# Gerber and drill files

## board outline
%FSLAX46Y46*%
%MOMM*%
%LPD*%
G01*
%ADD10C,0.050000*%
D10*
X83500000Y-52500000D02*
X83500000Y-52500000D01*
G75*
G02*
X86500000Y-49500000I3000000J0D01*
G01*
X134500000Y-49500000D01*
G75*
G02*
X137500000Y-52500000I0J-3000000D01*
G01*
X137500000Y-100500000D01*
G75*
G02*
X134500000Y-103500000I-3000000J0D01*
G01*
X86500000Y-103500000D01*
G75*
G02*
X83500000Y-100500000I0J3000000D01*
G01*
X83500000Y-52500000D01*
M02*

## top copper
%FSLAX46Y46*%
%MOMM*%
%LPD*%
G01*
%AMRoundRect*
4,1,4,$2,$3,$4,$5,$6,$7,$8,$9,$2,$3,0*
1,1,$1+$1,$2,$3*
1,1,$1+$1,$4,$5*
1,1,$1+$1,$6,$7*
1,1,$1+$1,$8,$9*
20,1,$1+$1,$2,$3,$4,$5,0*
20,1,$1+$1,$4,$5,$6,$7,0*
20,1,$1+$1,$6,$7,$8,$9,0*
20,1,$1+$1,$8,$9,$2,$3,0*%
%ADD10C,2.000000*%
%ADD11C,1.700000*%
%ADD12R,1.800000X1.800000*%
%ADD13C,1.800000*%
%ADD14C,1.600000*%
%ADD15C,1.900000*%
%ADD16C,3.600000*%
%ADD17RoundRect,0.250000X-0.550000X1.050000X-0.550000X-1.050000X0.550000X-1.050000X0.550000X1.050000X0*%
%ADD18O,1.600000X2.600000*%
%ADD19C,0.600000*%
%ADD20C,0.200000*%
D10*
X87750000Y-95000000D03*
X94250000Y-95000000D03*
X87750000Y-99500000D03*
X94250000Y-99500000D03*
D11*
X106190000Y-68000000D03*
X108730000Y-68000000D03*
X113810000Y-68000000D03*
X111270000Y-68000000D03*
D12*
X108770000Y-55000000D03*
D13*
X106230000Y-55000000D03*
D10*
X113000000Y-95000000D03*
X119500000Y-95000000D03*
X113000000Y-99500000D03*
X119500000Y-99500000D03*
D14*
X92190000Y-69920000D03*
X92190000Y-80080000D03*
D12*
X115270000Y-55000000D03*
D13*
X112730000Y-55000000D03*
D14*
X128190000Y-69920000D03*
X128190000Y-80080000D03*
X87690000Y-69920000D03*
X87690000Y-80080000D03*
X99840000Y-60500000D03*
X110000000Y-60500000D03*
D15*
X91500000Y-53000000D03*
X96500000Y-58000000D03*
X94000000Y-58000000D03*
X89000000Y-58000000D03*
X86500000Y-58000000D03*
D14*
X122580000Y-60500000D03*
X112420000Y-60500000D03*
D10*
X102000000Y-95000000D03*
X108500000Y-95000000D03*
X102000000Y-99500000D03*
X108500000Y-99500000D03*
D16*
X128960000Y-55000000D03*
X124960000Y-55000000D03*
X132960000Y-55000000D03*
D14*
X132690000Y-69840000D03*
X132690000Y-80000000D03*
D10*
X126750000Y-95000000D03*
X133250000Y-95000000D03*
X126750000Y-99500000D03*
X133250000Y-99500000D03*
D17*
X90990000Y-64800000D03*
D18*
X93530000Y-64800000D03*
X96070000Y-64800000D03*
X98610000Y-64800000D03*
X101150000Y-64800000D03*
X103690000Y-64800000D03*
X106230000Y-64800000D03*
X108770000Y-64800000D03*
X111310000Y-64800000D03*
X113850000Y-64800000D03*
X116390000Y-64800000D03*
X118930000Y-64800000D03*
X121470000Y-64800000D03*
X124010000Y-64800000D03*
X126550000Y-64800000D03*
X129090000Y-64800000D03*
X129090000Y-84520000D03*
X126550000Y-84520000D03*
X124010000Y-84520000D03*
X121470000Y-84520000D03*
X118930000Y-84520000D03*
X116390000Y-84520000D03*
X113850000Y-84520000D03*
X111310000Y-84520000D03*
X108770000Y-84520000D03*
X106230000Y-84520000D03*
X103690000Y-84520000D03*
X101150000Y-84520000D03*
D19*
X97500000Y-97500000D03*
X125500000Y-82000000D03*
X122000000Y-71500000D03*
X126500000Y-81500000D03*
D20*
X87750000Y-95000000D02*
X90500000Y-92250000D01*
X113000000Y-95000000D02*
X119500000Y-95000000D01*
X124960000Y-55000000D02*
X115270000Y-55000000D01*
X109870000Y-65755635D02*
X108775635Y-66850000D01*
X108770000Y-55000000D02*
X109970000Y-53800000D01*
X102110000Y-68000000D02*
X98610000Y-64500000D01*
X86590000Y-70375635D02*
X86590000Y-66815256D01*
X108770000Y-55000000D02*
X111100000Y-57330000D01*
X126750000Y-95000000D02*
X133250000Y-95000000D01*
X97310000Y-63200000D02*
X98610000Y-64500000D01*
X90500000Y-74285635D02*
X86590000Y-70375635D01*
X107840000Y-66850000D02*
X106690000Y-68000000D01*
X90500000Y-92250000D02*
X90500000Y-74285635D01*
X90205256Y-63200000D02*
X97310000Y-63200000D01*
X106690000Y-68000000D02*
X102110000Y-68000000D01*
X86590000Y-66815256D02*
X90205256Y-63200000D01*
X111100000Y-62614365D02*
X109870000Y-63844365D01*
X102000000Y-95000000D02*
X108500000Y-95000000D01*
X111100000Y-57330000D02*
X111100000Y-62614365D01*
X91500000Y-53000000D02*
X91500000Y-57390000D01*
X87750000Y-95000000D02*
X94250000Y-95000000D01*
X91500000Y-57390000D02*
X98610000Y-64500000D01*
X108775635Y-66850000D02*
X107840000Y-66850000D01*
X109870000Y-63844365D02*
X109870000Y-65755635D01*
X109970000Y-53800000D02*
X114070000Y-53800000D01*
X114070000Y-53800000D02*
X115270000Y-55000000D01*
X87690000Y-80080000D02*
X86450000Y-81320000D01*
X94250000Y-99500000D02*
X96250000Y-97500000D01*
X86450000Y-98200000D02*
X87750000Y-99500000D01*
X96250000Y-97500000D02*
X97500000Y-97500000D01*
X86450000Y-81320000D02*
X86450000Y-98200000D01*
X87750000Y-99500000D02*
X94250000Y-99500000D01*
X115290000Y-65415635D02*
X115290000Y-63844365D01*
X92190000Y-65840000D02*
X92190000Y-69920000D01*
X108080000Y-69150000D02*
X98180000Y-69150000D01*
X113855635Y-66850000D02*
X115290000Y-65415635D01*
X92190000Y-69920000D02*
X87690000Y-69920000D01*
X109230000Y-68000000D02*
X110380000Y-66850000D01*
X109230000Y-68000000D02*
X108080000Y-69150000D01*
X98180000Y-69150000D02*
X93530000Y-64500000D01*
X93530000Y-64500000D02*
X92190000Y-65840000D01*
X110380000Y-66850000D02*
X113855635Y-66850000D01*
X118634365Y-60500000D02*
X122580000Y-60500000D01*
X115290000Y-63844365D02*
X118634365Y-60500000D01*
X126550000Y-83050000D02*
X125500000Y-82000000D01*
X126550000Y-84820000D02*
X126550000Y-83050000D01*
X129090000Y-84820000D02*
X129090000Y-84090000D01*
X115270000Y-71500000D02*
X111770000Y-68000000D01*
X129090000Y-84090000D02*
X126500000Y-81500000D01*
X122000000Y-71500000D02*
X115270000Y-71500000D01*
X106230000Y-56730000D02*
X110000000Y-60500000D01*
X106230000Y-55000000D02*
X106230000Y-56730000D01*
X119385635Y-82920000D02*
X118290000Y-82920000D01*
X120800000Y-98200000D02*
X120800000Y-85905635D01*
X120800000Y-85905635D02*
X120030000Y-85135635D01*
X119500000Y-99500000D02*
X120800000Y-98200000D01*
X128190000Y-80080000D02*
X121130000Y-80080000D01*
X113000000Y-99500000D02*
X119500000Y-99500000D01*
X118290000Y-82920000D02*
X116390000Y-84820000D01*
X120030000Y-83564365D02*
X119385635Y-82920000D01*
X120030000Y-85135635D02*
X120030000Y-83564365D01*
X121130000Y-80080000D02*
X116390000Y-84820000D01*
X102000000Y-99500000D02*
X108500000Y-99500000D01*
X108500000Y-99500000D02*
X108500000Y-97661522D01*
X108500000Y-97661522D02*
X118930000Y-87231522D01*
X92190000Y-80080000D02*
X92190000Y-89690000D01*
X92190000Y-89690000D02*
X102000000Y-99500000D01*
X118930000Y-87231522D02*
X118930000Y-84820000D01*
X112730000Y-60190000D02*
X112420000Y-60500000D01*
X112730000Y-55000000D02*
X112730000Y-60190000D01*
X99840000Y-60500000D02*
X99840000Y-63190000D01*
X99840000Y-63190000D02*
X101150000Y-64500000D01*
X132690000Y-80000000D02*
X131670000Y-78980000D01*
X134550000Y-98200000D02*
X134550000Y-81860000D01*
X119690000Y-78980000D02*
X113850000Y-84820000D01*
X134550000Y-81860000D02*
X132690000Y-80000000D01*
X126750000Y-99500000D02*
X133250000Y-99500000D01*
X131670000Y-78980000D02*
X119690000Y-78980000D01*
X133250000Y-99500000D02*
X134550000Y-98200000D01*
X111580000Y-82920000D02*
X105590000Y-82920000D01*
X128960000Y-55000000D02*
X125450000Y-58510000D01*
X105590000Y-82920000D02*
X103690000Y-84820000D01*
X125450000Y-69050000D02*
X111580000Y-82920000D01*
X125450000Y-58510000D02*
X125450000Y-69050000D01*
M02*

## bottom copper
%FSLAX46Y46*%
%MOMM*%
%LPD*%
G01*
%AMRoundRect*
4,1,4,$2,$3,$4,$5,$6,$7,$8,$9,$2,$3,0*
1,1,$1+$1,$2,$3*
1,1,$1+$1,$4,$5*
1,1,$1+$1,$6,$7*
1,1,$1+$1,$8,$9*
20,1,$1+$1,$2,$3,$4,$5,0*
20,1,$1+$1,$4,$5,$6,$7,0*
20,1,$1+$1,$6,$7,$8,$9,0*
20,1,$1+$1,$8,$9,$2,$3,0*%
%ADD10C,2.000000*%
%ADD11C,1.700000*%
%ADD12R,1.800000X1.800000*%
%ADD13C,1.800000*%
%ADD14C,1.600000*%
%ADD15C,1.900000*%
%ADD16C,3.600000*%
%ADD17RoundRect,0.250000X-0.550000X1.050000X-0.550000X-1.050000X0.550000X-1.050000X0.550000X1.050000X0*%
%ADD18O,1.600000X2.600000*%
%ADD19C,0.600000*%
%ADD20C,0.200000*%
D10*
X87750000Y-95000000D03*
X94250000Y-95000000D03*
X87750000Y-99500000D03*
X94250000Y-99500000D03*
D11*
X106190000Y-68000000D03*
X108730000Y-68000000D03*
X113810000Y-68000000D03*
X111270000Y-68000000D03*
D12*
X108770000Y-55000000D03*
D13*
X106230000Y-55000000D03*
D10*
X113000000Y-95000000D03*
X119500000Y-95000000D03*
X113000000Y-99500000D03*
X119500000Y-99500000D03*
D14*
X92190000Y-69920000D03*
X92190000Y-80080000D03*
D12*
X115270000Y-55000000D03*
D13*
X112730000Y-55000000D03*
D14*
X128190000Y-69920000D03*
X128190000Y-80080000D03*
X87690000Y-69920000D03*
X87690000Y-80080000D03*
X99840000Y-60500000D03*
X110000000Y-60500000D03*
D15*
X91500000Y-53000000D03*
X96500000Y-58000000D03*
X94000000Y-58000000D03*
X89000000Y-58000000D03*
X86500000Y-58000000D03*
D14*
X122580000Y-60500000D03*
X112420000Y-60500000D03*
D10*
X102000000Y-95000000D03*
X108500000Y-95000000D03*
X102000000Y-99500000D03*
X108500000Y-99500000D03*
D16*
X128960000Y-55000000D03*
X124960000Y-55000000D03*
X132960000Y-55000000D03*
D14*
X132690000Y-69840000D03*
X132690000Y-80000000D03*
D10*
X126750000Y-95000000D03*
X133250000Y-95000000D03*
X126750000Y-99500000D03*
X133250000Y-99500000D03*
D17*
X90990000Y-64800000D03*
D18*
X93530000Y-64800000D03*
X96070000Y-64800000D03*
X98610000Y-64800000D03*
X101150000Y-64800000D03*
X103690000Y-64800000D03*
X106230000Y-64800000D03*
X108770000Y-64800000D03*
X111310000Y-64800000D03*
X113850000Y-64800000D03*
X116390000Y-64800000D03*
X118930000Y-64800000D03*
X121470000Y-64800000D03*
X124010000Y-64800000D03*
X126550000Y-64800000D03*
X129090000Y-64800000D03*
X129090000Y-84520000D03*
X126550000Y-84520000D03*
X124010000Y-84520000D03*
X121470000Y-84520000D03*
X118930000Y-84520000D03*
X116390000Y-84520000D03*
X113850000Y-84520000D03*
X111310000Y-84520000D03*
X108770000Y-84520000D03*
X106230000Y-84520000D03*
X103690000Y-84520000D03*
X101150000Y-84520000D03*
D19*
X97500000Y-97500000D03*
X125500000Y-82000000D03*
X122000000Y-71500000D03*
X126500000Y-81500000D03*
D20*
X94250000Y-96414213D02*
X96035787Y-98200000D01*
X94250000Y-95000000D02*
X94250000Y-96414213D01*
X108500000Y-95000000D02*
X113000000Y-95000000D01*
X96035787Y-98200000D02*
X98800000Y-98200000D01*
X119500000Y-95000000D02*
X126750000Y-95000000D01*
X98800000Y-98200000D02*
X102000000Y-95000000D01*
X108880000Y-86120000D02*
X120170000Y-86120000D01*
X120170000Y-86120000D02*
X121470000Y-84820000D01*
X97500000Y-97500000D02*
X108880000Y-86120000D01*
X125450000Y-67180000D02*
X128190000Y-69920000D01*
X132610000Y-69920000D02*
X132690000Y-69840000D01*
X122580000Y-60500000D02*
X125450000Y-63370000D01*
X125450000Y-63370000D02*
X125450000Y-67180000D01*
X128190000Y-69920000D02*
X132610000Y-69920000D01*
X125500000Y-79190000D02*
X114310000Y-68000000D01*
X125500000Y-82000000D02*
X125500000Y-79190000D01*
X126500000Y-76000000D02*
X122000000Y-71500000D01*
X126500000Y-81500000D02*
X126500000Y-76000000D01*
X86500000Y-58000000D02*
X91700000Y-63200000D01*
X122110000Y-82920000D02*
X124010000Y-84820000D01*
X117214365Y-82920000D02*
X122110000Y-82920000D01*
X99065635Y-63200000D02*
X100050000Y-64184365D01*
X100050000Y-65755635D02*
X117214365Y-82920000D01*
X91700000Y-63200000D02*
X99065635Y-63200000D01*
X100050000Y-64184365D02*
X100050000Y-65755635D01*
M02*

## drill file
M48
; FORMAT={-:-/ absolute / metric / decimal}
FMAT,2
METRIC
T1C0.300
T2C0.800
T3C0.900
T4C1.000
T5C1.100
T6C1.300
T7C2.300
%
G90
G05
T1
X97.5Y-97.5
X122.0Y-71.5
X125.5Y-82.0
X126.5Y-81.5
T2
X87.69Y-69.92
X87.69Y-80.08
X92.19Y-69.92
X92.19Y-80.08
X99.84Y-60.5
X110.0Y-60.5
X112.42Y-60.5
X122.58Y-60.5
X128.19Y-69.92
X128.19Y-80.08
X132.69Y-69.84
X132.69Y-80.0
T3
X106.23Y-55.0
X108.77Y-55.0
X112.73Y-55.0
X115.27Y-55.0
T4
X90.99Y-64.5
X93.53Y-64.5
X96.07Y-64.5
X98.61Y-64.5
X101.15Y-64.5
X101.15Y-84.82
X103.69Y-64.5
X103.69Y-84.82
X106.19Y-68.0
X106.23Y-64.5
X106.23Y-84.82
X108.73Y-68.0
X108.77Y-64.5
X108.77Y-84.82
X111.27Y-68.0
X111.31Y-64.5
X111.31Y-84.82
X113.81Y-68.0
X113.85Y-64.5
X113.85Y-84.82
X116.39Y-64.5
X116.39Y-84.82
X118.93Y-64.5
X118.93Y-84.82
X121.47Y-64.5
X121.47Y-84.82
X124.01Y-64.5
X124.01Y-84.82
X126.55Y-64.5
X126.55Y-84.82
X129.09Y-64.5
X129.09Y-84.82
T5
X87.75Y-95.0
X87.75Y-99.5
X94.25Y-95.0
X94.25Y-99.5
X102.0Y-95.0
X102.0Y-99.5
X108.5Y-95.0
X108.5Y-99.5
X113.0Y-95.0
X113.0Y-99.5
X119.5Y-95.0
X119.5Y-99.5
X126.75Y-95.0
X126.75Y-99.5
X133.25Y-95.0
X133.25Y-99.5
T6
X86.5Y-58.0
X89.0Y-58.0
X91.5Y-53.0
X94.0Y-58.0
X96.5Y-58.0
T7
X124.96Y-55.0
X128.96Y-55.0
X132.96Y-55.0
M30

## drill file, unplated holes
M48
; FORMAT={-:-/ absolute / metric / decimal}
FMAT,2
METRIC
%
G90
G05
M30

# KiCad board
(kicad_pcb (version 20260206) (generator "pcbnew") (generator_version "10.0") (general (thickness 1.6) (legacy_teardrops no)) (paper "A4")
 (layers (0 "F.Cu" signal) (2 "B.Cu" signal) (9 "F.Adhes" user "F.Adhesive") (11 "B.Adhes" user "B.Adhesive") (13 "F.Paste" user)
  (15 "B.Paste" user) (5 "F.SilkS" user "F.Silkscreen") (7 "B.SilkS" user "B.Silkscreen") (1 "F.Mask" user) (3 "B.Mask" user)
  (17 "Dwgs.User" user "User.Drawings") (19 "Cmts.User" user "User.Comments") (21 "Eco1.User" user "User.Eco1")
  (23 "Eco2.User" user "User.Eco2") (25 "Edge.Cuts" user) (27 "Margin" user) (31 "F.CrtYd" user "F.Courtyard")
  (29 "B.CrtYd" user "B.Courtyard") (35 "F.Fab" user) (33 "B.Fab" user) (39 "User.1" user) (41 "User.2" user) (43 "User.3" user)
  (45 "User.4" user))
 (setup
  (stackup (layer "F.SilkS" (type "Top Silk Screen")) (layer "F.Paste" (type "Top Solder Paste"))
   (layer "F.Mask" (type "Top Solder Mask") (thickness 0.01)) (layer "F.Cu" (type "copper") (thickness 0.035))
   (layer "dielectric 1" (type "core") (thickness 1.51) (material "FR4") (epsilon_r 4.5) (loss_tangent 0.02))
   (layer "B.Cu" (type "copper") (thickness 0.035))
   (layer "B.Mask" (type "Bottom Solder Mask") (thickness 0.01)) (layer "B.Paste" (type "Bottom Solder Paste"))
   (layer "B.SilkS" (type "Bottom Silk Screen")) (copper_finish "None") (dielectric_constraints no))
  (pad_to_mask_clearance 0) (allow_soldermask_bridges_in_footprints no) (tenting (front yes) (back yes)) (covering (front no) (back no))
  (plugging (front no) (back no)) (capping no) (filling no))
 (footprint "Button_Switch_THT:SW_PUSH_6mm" (layer "F.Cu") (at 87.75 95)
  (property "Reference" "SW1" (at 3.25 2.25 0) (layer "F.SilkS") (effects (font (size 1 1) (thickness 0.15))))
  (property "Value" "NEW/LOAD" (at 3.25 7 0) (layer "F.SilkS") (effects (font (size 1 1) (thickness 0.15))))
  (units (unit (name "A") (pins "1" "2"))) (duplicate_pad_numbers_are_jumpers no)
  (pad "1" thru_hole circle (at 0 0 90) (size 2 2) (drill 1.1) (layers "*.Cu" "*.Mask") (remove_unused_layers no) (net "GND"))
  (pad "1" thru_hole circle (at 6.5 0 90) (size 2 2) (drill 1.1) (layers "*.Cu" "*.Mask") (remove_unused_layers no) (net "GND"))
  (pad "2" thru_hole circle (at 0 4.5 90) (size 2 2) (drill 1.1) (layers "*.Cu" "*.Mask") (remove_unused_layers no) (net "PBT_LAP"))
  (pad "2" thru_hole circle (at 6.5 4.5 90) (size 2 2) (drill 1.1) (layers "*.Cu" "*.Mask") (remove_unused_layers no) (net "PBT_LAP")))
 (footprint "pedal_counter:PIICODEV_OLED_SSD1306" (layer "F.Cu") (at 110 80)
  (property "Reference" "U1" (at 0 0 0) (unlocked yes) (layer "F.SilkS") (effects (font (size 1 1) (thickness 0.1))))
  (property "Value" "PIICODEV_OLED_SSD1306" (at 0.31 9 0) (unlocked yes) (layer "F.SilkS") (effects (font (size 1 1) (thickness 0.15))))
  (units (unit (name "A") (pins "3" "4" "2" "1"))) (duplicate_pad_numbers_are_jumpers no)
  (pad "1" thru_hole circle (at -3.81 -12) (size 1.7 1.7) (drill 1) (layers "*.Cu" "*.Mask") (remove_unused_layers no) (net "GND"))
  (pad "2" thru_hole circle (at -1.27 -12) (size 1.7 1.7) (drill 1) (layers "*.Cu" "*.Mask") (remove_unused_layers no) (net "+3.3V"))
  (pad "3" thru_hole circle (at 3.81 -12) (size 1.7 1.7) (drill 1) (layers "*.Cu" "*.Mask") (remove_unused_layers no) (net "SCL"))
  (pad "4" thru_hole circle (at 1.27 -12) (size 1.7 1.7) (drill 1) (layers "*.Cu" "*.Mask") (remove_unused_layers no) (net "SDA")))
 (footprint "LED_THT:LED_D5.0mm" (layer "F.Cu") (at 108.77 55 180)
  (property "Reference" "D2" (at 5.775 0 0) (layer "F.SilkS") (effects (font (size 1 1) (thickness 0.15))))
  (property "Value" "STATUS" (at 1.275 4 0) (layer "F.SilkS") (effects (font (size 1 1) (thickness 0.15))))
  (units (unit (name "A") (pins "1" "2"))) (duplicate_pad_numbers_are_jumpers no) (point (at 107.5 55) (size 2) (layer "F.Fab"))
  (pad "1" thru_hole rect (at 0 0 180) (size 1.8 1.8) (drill 0.9) (layers "*.Cu" "*.Mask") (remove_unused_layers no) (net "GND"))
  (pad "2" thru_hole circle (at 2.54 0 180) (size 1.8 1.8) (drill 0.9) (layers "*.Cu" "*.Mask") (remove_unused_layers no) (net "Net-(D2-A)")))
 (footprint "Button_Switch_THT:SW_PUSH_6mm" (layer "F.Cu") (at 113 95)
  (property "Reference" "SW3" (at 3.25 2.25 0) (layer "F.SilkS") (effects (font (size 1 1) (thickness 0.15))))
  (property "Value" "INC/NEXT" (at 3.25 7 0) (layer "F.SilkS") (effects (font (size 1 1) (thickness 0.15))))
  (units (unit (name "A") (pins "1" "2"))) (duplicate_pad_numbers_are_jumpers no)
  (pad "1" thru_hole circle (at 0 0 90) (size 2 2) (drill 1.1) (layers "*.Cu" "*.Mask") (remove_unused_layers no) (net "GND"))
  (pad "1" thru_hole circle (at 6.5 0 90) (size 2 2) (drill 1.1) (layers "*.Cu" "*.Mask") (remove_unused_layers no) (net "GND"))
  (pad "2" thru_hole circle (at 0 4.5 90) (size 2 2) (drill 1.1) (layers "*.Cu" "*.Mask") (remove_unused_layers no) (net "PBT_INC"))
  (pad "2" thru_hole circle (at 6.5 4.5 90) (size 2 2) (drill 1.1) (layers "*.Cu" "*.Mask") (remove_unused_layers no) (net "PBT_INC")))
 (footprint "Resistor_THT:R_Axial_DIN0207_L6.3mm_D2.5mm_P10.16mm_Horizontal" (layer "F.Cu") (at 92.19 69.92 -90)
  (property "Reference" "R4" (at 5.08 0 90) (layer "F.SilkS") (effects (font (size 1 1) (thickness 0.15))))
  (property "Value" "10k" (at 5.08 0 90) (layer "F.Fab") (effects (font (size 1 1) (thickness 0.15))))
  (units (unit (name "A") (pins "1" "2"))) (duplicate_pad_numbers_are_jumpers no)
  (pad "1" thru_hole circle (at 0 0 270) (size 1.6 1.6) (drill 0.8) (layers "*.Cu" "*.Mask") (remove_unused_layers no) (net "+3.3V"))
  (pad "2" thru_hole circle (at 10.16 0 270) (size 1.6 1.6) (drill 0.8) (layers "*.Cu" "*.Mask") (remove_unused_layers no) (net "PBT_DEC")))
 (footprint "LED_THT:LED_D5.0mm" (layer "F.Cu") (at 115.27 55 180)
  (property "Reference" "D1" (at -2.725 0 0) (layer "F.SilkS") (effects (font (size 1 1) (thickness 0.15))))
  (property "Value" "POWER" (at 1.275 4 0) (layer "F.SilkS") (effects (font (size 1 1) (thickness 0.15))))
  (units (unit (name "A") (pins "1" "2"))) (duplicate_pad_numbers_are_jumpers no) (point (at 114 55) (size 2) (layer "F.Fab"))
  (pad "1" thru_hole rect (at 0 0 180) (size 1.8 1.8) (drill 0.9) (layers "*.Cu" "*.Mask") (remove_unused_layers no) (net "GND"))
  (pad "2" thru_hole circle (at 2.54 0 180) (size 1.8 1.8) (drill 0.9) (layers "*.Cu" "*.Mask") (remove_unused_layers no) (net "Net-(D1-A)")))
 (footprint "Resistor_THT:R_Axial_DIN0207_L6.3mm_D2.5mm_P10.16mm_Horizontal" (layer "F.Cu") (at 128.19 69.92 -90)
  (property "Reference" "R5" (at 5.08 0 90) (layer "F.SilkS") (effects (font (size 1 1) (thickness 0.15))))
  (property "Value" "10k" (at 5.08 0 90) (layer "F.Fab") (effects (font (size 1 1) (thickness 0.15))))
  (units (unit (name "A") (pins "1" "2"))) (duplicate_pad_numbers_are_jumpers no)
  (pad "1" thru_hole circle (at 0 0 270) (size 1.6 1.6) (drill 0.8) (layers "*.Cu" "*.Mask") (remove_unused_layers no) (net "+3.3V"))
  (pad "2" thru_hole circle (at 10.16 0 270) (size 1.6 1.6) (drill 0.8) (layers "*.Cu" "*.Mask") (remove_unused_layers no) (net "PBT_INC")))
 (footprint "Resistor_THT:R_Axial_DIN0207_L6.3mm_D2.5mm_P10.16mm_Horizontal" (layer "F.Cu") (at 87.69 69.92 -90)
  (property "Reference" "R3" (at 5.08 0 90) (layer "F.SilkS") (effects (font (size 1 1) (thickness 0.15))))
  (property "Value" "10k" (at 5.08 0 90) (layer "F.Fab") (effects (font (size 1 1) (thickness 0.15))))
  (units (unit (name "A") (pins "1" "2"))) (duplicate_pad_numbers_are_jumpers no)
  (pad "1" thru_hole circle (at 0 0 270) (size 1.6 1.6) (drill 0.8) (layers "*.Cu" "*.Mask") (remove_unused_layers no) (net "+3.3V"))
  (pad "2" thru_hole circle (at 10.16 0 270) (size 1.6 1.6) (drill 0.8) (layers "*.Cu" "*.Mask") (remove_unused_layers no) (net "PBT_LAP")))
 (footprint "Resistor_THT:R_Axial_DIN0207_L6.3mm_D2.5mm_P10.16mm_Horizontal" (layer "F.Cu") (at 99.84 60.5)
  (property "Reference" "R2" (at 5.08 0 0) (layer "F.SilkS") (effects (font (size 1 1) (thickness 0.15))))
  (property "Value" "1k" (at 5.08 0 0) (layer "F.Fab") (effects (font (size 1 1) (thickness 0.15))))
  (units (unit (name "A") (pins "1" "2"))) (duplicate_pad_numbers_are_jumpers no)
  (pad "1" thru_hole circle (at 0 0) (size 1.6 1.6) (drill 0.8) (layers "*.Cu" "*.Mask") (remove_unused_layers no) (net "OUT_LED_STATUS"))
  (pad "2" thru_hole circle (at 10.16 0) (size 1.6 1.6) (drill 0.8) (layers "*.Cu" "*.Mask") (remove_unused_layers no) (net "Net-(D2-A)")))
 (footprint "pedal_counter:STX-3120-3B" (layer "F.Cu") (at 91.5 58 -90)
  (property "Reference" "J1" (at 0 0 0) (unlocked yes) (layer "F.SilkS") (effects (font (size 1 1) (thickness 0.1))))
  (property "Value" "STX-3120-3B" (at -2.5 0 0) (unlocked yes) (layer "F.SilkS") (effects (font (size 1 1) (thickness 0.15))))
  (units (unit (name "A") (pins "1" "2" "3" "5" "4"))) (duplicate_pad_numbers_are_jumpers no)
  (pad "1" thru_hole circle (at -5 0 270) (size 1.9 1.9) (drill 1.3) (layers "*.Cu" "*.Mask") (remove_unused_layers no) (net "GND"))
  (pad "2" thru_hole circle (at 0 -5 270) (size 1.9 1.9) (drill 1.3) (layers "*.Cu" "*.Mask") (remove_unused_layers no)
   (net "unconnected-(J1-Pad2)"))
  (pad "3" thru_hole circle (at 0 -2.5 270) (size 1.9 1.9) (drill 1.3) (layers "*.Cu" "*.Mask") (remove_unused_layers no)
   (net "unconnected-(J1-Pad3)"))
  (pad "4" thru_hole circle (at 0 2.5 270) (size 1.9 1.9) (drill 1.3) (layers "*.Cu" "*.Mask") (remove_unused_layers no)
   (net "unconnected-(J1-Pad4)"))
  (pad "5" thru_hole circle (at 0 5 270) (size 1.9 1.9) (drill 1.3) (layers "*.Cu" "*.Mask") (remove_unused_layers no) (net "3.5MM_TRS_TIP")))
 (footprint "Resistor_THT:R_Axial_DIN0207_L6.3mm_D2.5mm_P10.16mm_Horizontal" (layer "F.Cu") (at 122.58 60.5 180)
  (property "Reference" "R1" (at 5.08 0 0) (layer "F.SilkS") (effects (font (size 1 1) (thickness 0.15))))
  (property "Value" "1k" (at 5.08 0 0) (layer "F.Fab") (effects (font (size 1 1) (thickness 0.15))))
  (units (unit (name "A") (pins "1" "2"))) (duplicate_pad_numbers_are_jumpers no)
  (pad "1" thru_hole circle (at 0 0 180) (size 1.6 1.6) (drill 0.8) (layers "*.Cu" "*.Mask") (remove_unused_layers no) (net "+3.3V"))
  (pad "2" thru_hole circle (at 10.16 0 180) (size 1.6 1.6) (drill 0.8) (layers "*.Cu" "*.Mask") (remove_unused_layers no)
   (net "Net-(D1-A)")))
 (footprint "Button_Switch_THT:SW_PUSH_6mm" (layer "F.Cu") (at 102 95)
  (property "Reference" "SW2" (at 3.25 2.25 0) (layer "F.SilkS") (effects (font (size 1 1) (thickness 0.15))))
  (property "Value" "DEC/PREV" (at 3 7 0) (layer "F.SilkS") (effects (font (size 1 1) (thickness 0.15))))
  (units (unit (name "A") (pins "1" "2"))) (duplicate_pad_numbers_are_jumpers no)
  (pad "1" thru_hole circle (at 0 0 90) (size 2 2) (drill 1.1) (layers "*.Cu" "*.Mask") (remove_unused_layers no) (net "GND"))
  (pad "1" thru_hole circle (at 6.5 0 90) (size 2 2) (drill 1.1) (layers "*.Cu" "*.Mask") (remove_unused_layers no) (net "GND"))
  (pad "2" thru_hole circle (at 0 4.5 90) (size 2 2) (drill 1.1) (layers "*.Cu" "*.Mask") (remove_unused_layers no) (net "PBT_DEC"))
  (pad "2" thru_hole circle (at 6.5 4.5 90) (size 2 2) (drill 1.1) (layers "*.Cu" "*.Mask") (remove_unused_layers no) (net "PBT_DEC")))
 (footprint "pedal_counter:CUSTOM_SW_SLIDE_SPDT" (layer "F.Cu") (at 128.96 55)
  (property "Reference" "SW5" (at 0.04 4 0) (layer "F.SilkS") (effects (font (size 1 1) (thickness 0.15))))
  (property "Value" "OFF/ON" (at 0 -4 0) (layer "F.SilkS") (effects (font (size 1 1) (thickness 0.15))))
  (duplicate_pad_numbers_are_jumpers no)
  (pad "1" thru_hole circle (at 0 0) (size 3.6 3.6) (drill 2.3) (layers "*.Cu" "*.Mask") (remove_unused_layers no) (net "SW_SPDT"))
  (pad "2" thru_hole circle (at -4 0) (size 3.6 3.6) (drill 2.3) (layers "*.Cu" "*.Mask") (remove_unused_layers no) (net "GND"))
  (pad "3" thru_hole circle (at 4 0) (size 3.6 3.6) (drill 2.3) (layers "*.Cu" "*.Mask") (remove_unused_layers no)
   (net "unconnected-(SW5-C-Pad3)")))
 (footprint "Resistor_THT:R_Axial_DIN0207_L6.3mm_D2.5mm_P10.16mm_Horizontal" (layer "F.Cu") (at 132.69 69.84 -90)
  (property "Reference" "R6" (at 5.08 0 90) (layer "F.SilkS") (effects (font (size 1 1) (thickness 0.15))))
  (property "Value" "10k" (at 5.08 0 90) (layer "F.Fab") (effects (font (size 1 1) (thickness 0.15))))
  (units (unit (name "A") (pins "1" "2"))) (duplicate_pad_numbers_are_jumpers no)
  (pad "1" thru_hole circle (at 0 0 270) (size 1.6 1.6) (drill 0.8) (layers "*.Cu" "*.Mask") (remove_unused_layers no) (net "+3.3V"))
  (pad "2" thru_hole circle (at 10.16 0 270) (size 1.6 1.6) (drill 0.8) (layers "*.Cu" "*.Mask") (remove_unused_layers no) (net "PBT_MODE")))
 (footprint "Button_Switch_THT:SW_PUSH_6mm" (layer "F.Cu") (at 126.75 95)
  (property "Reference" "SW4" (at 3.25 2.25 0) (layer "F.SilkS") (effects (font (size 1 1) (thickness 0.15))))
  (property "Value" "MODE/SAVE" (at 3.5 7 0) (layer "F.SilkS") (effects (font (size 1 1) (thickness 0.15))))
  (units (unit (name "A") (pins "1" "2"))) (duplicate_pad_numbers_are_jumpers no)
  (pad "1" thru_hole circle (at 0 0 90) (size 2 2) (drill 1.1) (layers "*.Cu" "*.Mask") (remove_unused_layers no) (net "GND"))
  (pad "1" thru_hole circle (at 6.5 0 90) (size 2 2) (drill 1.1) (layers "*.Cu" "*.Mask") (remove_unused_layers no) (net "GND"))
  (pad "2" thru_hole circle (at 0 4.5 90) (size 2 2) (drill 1.1) (layers "*.Cu" "*.Mask") (remove_unused_layers no) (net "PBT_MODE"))
  (pad "2" thru_hole circle (at 6.5 4.5 90) (size 2 2) (drill 1.1) (layers "*.Cu" "*.Mask") (remove_unused_layers no) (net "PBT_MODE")))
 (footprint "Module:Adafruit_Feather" (layer "B.Cu") (at 90.99 64.5 -90)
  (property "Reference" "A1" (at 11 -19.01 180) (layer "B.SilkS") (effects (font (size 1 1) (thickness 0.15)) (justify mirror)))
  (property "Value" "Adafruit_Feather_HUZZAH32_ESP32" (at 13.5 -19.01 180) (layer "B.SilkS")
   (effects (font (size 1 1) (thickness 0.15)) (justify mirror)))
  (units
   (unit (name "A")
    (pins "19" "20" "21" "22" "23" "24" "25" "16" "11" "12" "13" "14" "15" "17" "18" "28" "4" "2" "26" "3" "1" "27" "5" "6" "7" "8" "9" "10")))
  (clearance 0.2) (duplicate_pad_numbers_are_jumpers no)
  (pad "1" thru_hole roundrect (at 0 0 270) (size 2.6 1.6) (drill 1 (offset 0.3 0)) (layers "*.Cu" "*.Mask") (remove_unused_layers no)
   (roundrect_rratio 0.15625) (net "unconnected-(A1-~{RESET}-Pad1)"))
  (pad "2" thru_hole oval (at 0 -2.54 270) (size 2.6 1.6) (drill 1 (offset 0.3 0)) (layers "*.Cu" "*.Mask") (remove_unused_layers no)
   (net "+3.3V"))
  (pad "3" thru_hole oval (at 0 -5.08 270) (size 2.6 1.6) (drill 1 (offset 0.3 0)) (layers "*.Cu" "*.Mask") (remove_unused_layers no)
   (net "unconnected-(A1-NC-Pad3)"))
  (pad "4" thru_hole oval (at 0 -7.62 270) (size 2.6 1.6) (drill 1 (offset 0.3 0)) (layers "*.Cu" "*.Mask") (remove_unused_layers no)
   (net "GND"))
  (pad "5" thru_hole oval (at 0 -10.16 270) (size 2.6 1.6) (drill 1 (offset 0.3 0)) (layers "*.Cu" "*.Mask") (remove_unused_layers no)
   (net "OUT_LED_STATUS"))
  (pad "6" thru_hole oval (at 0 -12.7 270) (size 2.6 1.6) (drill 1 (offset 0.3 0)) (layers "*.Cu" "*.Mask") (remove_unused_layers no)
   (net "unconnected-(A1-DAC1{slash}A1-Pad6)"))
  (pad "7" thru_hole oval (at 0 -15.24 270) (size 2.6 1.6) (drill 1 (offset 0.3 0)) (layers "*.Cu" "*.Mask") (remove_unused_layers no)
   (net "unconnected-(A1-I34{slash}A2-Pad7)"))
  (pad "8" thru_hole oval (at 0 -17.78 270) (size 2.6 1.6) (drill 1 (offset 0.3 0)) (layers "*.Cu" "*.Mask") (remove_unused_layers no)
   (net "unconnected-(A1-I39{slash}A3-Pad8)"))
  (pad "9" thru_hole oval (at 0 -20.32 270) (size 2.6 1.6) (drill 1 (offset 0.3 0)) (layers "*.Cu" "*.Mask") (remove_unused_layers no)
   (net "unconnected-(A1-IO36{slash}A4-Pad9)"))
  (pad "10" thru_hole oval (at 0 -22.86 270) (size 2.6 1.6) (drill 1 (offset 0.3 0)) (layers "*.Cu" "*.Mask") (remove_unused_layers no)
   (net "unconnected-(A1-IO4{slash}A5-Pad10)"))
  (pad "11" thru_hole oval (at 0 -25.4 270) (size 2.6 1.6) (drill 1 (offset 0.3 0)) (layers "*.Cu" "*.Mask") (remove_unused_layers no)
   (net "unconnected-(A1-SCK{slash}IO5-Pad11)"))
  (pad "12" thru_hole oval (at 0 -27.94 270) (size 2.6 1.6) (drill 1 (offset 0.3 0)) (layers "*.Cu" "*.Mask") (remove_unused_layers no)
   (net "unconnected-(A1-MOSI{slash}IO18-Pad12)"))
  (pad "13" thru_hole oval (at 0 -30.48 270) (size 2.6 1.6) (drill 1 (offset 0.3 0)) (layers "*.Cu" "*.Mask") (remove_unused_layers no)
   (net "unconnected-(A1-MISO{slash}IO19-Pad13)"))
  (pad "14" thru_hole oval (at 0 -33.02 270) (size 2.6 1.6) (drill 1 (offset 0.3 0)) (layers "*.Cu" "*.Mask") (remove_unused_layers no)
   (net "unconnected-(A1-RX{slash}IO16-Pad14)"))
  (pad "15" thru_hole oval (at 0 -35.56 270) (size 2.6 1.6) (drill 1 (offset 0.3 0)) (layers "*.Cu" "*.Mask") (remove_unused_layers no)
   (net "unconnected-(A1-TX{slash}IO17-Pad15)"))
  (pad "16" thru_hole oval (at 0 -38.1 270) (size 2.6 1.6) (drill 1 (offset 0.3 0)) (layers "*.Cu" "*.Mask") (remove_unused_layers no)
   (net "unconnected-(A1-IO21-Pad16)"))
  (pad "17" thru_hole oval (at 20.32 -38.1 90) (size 2.6 1.6) (drill 1 (offset 0.3 0)) (layers "*.Cu" "*.Mask") (remove_unused_layers no)
   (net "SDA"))
  (pad "18" thru_hole oval (at 20.32 -35.56 90) (size 2.6 1.6) (drill 1 (offset 0.3 0)) (layers "*.Cu" "*.Mask") (remove_unused_layers no)
   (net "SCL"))
  (pad "19" thru_hole oval (at 20.32 -33.02 90) (size 2.6 1.6) (drill 1 (offset 0.3 0)) (layers "*.Cu" "*.Mask") (remove_unused_layers no)
   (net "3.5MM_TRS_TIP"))
  (pad "20" thru_hole oval (at 20.32 -30.48 90) (size 2.6 1.6) (drill 1 (offset 0.3 0)) (layers "*.Cu" "*.Mask") (remove_unused_layers no)
   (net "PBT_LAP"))
  (pad "21" thru_hole oval (at 20.32 -27.94 90) (size 2.6 1.6) (drill 1 (offset 0.3 0)) (layers "*.Cu" "*.Mask") (remove_unused_layers no)
   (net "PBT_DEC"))
  (pad "22" thru_hole oval (at 20.32 -25.4 90) (size 2.6 1.6) (drill 1 (offset 0.3 0)) (layers "*.Cu" "*.Mask") (remove_unused_layers no)
   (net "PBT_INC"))
  (pad "23" thru_hole oval (at 20.32 -22.86 90) (size 2.6 1.6) (drill 1 (offset 0.3 0)) (layers "*.Cu" "*.Mask") (remove_unused_layers no)
   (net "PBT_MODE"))
  (pad "24" thru_hole oval (at 20.32 -20.32 90) (size 2.6 1.6) (drill 1 (offset 0.3 0)) (layers "*.Cu" "*.Mask") (remove_unused_layers no)
   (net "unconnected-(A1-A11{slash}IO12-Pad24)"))
  (pad "25" thru_hole oval (at 20.32 -17.78 90) (size 2.6 1.6) (drill 1 (offset 0.3 0)) (layers "*.Cu" "*.Mask") (remove_unused_layers no)
   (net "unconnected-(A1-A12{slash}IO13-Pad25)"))
  (pad "26" thru_hole oval (at 20.32 -15.24 90) (size 2.6 1.6) (drill 1 (offset 0.3 0)) (layers "*.Cu" "*.Mask") (remove_unused_layers no)
   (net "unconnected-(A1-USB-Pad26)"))
  (pad "27" thru_hole oval (at 20.32 -12.7 90) (size 2.6 1.6) (drill 1 (offset 0.3 0)) (layers "*.Cu" "*.Mask") (remove_unused_layers no)
   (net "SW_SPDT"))
  (pad "28" thru_hole oval (at 20.32 -10.16 90) (size 2.6 1.6) (drill 1 (offset 0.3 0)) (layers "*.Cu" "*.Mask") (remove_unused_layers no)
   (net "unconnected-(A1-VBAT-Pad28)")))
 (gr_rect (start 83.5 49.5) (end 137.5 103.5) (radius 3) (stroke (width 0.05) (type solid)) (fill no) (layer "Edge.Cuts"))
 (segment (start 87.75 95) (end 90.5 92.25) (width 0.2) (layer "F.Cu") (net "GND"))
 (segment (start 113 95) (end 119.5 95) (width 0.2) (layer "F.Cu") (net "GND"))
 (segment (start 124.96 55) (end 115.27 55) (width 0.2) (layer "F.Cu") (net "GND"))
 (segment (start 109.87 65.755635) (end 108.775635 66.85) (width 0.2) (layer "F.Cu") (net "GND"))
 (segment (start 108.77 55) (end 109.97 53.8) (width 0.2) (layer "F.Cu") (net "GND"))
 (segment (start 102.11 68) (end 98.61 64.5) (width 0.2) (layer "F.Cu") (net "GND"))
 (segment (start 86.59 70.375635) (end 86.59 66.815256) (width 0.2) (layer "F.Cu") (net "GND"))
 (segment (start 108.77 55) (end 111.1 57.33) (width 0.2) (layer "F.Cu") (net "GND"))
 (segment (start 126.75 95) (end 133.25 95) (width 0.2) (layer "F.Cu") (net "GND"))
 (segment (start 97.31 63.2) (end 98.61 64.5) (width 0.2) (layer "F.Cu") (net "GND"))
 (segment (start 90.5 74.285635) (end 86.59 70.375635) (width 0.2) (layer "F.Cu") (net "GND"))
 (segment (start 107.84 66.85) (end 106.69 68) (width 0.2) (layer "F.Cu") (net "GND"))
 (segment (start 90.5 92.25) (end 90.5 74.285635) (width 0.2) (layer "F.Cu") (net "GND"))
 (segment (start 90.205256 63.2) (end 97.31 63.2) (width 0.2) (layer "F.Cu") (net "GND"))
 (segment (start 106.69 68) (end 102.11 68) (width 0.2) (layer "F.Cu") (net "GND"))
 (segment (start 86.59 66.815256) (end 90.205256 63.2) (width 0.2) (layer "F.Cu") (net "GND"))
 (segment (start 111.1 62.614365) (end 109.87 63.844365) (width 0.2) (layer "F.Cu") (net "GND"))
 (segment (start 102 95) (end 108.5 95) (width 0.2) (layer "F.Cu") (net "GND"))
 (segment (start 111.1 57.33) (end 111.1 62.614365) (width 0.2) (layer "F.Cu") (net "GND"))
 (segment (start 91.5 53) (end 91.5 57.39) (width 0.2) (layer "F.Cu") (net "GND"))
 (segment (start 87.75 95) (end 94.25 95) (width 0.2) (layer "F.Cu") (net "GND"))
 (segment (start 91.5 57.39) (end 98.61 64.5) (width 0.2) (layer "F.Cu") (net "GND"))
 (segment (start 108.775635 66.85) (end 107.84 66.85) (width 0.2) (layer "F.Cu") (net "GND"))
 (segment (start 109.87 63.844365) (end 109.87 65.755635) (width 0.2) (layer "F.Cu") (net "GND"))
 (segment (start 109.97 53.8) (end 114.07 53.8) (width 0.2) (layer "F.Cu") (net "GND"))
 (segment (start 114.07 53.8) (end 115.27 55) (width 0.2) (layer "F.Cu") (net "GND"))
 (segment (start 94.25 96.414213) (end 96.035787 98.2) (width 0.2) (layer "B.Cu") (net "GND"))
 (segment (start 94.25 95) (end 94.25 96.414213) (width 0.2) (layer "B.Cu") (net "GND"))
 (segment (start 108.5 95) (end 113 95) (width 0.2) (layer "B.Cu") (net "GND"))
 (segment (start 96.035787 98.2) (end 98.8 98.2) (width 0.2) (layer "B.Cu") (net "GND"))
 (segment (start 119.5 95) (end 126.75 95) (width 0.2) (layer "B.Cu") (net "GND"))
 (segment (start 98.8 98.2) (end 102 95) (width 0.2) (layer "B.Cu") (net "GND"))
 (segment (start 87.69 80.08) (end 86.45 81.32) (width 0.2) (layer "F.Cu") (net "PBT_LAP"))
 (segment (start 94.25 99.5) (end 96.25 97.5) (width 0.2) (layer "F.Cu") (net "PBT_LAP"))
 (segment (start 86.45 98.2) (end 87.75 99.5) (width 0.2) (layer "F.Cu") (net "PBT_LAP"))
 (segment (start 96.25 97.5) (end 97.5 97.5) (width 0.2) (layer "F.Cu") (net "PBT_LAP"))
 (segment (start 86.45 81.32) (end 86.45 98.2) (width 0.2) (layer "F.Cu") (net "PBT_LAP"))
 (segment (start 87.75 99.5) (end 94.25 99.5) (width 0.2) (layer "F.Cu") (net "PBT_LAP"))
 (via (at 97.5 97.5) (size 0.6) (drill 0.3) (layers "F.Cu" "B.Cu") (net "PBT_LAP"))
 (segment (start 108.88 86.12) (end 120.17 86.12) (width 0.2) (layer "B.Cu") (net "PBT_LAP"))
 (segment (start 120.17 86.12) (end 121.47 84.82) (width 0.2) (layer "B.Cu") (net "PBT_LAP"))
 (segment (start 97.5 97.5) (end 108.88 86.12) (width 0.2) (layer "B.Cu") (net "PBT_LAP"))
 (segment (start 115.29 65.415635) (end 115.29 63.844365) (width 0.2) (layer "F.Cu") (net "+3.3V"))
 (segment (start 92.19 65.84) (end 92.19 69.92) (width 0.2) (layer "F.Cu") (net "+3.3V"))
 (segment (start 108.08 69.15) (end 98.18 69.15) (width 0.2) (layer "F.Cu") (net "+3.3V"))
 (segment (start 113.855635 66.85) (end 115.29 65.415635) (width 0.2) (layer "F.Cu") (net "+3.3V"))
 (segment (start 92.19 69.92) (end 87.69 69.92) (width 0.2) (layer "F.Cu") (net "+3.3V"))
 (segment (start 109.23 68) (end 110.38 66.85) (width 0.2) (layer "F.Cu") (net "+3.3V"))
 (segment (start 109.23 68) (end 108.08 69.15) (width 0.2) (layer "F.Cu") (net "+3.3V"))
 (segment (start 98.18 69.15) (end 93.53 64.5) (width 0.2) (layer "F.Cu") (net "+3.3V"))
 (segment (start 93.53 64.5) (end 92.19 65.84) (width 0.2) (layer "F.Cu") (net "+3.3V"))
 (segment (start 110.38 66.85) (end 113.855635 66.85) (width 0.2) (layer "F.Cu") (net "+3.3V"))
 (segment (start 118.634365 60.5) (end 122.58 60.5) (width 0.2) (layer "F.Cu") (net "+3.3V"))
 (segment (start 115.29 63.844365) (end 118.634365 60.5) (width 0.2) (layer "F.Cu") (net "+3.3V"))
 (segment (start 125.45 67.18) (end 128.19 69.92) (width 0.2) (layer "B.Cu") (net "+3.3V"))
 (segment (start 132.61 69.92) (end 132.69 69.84) (width 0.2) (layer "B.Cu") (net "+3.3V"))
 (segment (start 122.58 60.5) (end 125.45 63.37) (width 0.2) (layer "B.Cu") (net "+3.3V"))
 (segment (start 125.45 63.37) (end 125.45 67.18) (width 0.2) (layer "B.Cu") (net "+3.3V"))
 (segment (start 128.19 69.92) (end 132.61 69.92) (width 0.2) (layer "B.Cu") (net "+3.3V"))
 (segment (start 126.55 83.05) (end 125.5 82) (width 0.2) (layer "F.Cu") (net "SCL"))
 (segment (start 126.55 84.82) (end 126.55 83.05) (width 0.2) (layer "F.Cu") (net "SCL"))
 (via (at 125.5 82) (size 0.6) (drill 0.3) (layers "F.Cu" "B.Cu") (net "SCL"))
 (segment (start 125.5 79.19) (end 114.31 68) (width 0.2) (layer "B.Cu") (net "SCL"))
 (segment (start 125.5 82) (end 125.5 79.19) (width 0.2) (layer "B.Cu") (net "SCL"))
 (segment (start 129.09 84.82) (end 129.09 84.09) (width 0.2) (layer "F.Cu") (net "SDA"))
 (segment (start 115.27 71.5) (end 111.77 68) (width 0.2) (layer "F.Cu") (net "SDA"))
 (segment (start 129.09 84.09) (end 126.5 81.5) (width 0.2) (layer "F.Cu") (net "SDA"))
 (segment (start 122 71.5) (end 115.27 71.5) (width 0.2) (layer "F.Cu") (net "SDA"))
 (via (at 122 71.5) (size 0.6) (drill 0.3) (layers "F.Cu" "B.Cu") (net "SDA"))
 (via (at 126.5 81.5) (size 0.6) (drill 0.3) (layers "F.Cu" "B.Cu") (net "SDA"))
 (segment (start 126.5 76) (end 122 71.5) (width 0.2) (layer "B.Cu") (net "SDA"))
 (segment (start 126.5 81.5) (end 126.5 76) (width 0.2) (layer "B.Cu") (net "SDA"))
 (segment (start 106.23 56.73) (end 110 60.5) (width 0.2) (layer "F.Cu") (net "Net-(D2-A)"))
 (segment (start 106.23 55) (end 106.23 56.73) (width 0.2) (layer "F.Cu") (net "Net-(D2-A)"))
 (segment (start 119.385635 82.92) (end 118.29 82.92) (width 0.2) (layer "F.Cu") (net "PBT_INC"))
 (segment (start 120.8 98.2) (end 120.8 85.905635) (width 0.2) (layer "F.Cu") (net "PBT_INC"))
 (segment (start 120.8 85.905635) (end 120.03 85.135635) (width 0.2) (layer "F.Cu") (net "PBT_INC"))
 (segment (start 119.5 99.5) (end 120.8 98.2) (width 0.2) (layer "F.Cu") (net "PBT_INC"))
 (segment (start 128.19 80.08) (end 121.13 80.08) (width 0.2) (layer "F.Cu") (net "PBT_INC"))
 (segment (start 113 99.5) (end 119.5 99.5) (width 0.2) (layer "F.Cu") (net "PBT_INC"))
 (segment (start 118.29 82.92) (end 116.39 84.82) (width 0.2) (layer "F.Cu") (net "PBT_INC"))
 (segment (start 120.03 83.564365) (end 119.385635 82.92) (width 0.2) (layer "F.Cu") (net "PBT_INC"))
 (segment (start 120.03 85.135635) (end 120.03 83.564365) (width 0.2) (layer "F.Cu") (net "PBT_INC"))
 (segment (start 121.13 80.08) (end 116.39 84.82) (width 0.2) (layer "F.Cu") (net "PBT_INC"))
 (segment (start 102 99.5) (end 108.5 99.5) (width 0.2) (layer "F.Cu") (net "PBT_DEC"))
 (segment (start 108.5 99.5) (end 108.5 97.661522) (width 0.2) (layer "F.Cu") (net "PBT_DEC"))
 (segment (start 108.5 97.661522) (end 118.93 87.231522) (width 0.2) (layer "F.Cu") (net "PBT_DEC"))
 (segment (start 92.19 80.08) (end 92.19 89.69) (width 0.2) (layer "F.Cu") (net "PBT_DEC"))
 (segment (start 92.19 89.69) (end 102 99.5) (width 0.2) (layer "F.Cu") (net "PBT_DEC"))
 (segment (start 118.93 87.231522) (end 118.93 84.82) (width 0.2) (layer "F.Cu") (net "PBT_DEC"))
 (segment (start 112.73 60.19) (end 112.42 60.5) (width 0.2) (layer "F.Cu") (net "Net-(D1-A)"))
 (segment (start 112.73 55) (end 112.73 60.19) (width 0.2) (layer "F.Cu") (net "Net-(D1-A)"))
 (segment (start 99.84 60.5) (end 99.84 63.19) (width 0.2) (layer "F.Cu") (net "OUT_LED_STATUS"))
 (segment (start 99.84 63.19) (end 101.15 64.5) (width 0.2) (layer "F.Cu") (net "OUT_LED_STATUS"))
 (segment (start 86.5 58) (end 91.7 63.2) (width 0.2) (layer "B.Cu") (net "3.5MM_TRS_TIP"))
 (segment (start 122.11 82.92) (end 124.01 84.82) (width 0.2) (layer "B.Cu") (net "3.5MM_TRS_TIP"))
 (segment (start 117.214365 82.92) (end 122.11 82.92) (width 0.2) (layer "B.Cu") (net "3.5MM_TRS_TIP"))
 (segment (start 99.065635 63.2) (end 100.05 64.184365) (width 0.2) (layer "B.Cu") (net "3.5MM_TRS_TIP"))
 (segment (start 100.05 65.755635) (end 117.214365 82.92) (width 0.2) (layer "B.Cu") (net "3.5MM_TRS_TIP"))
 (segment (start 91.7 63.2) (end 99.065635 63.2) (width 0.2) (layer "B.Cu") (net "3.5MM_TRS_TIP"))
 (segment (start 100.05 64.184365) (end 100.05 65.755635) (width 0.2) (layer "B.Cu") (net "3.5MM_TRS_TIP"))
 (segment (start 111.58 82.92) (end 105.59 82.92) (width 0.2) (layer "F.Cu") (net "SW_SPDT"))
 (segment (start 128.96 55) (end 125.45 58.51) (width 0.2) (layer "F.Cu") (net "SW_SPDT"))
 (segment (start 105.59 82.92) (end 103.69 84.82) (width 0.2) (layer "F.Cu") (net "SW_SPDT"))
 (segment (start 125.45 69.05) (end 111.58 82.92) (width 0.2) (layer "F.Cu") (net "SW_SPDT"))
 (segment (start 125.45 58.51) (end 125.45 69.05) (width 0.2) (layer "F.Cu") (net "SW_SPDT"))
 (segment (start 132.69 80) (end 131.67 78.98) (width 0.2) (layer "F.Cu") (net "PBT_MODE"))
 (segment (start 134.55 98.2) (end 134.55 81.86) (width 0.2) (layer "F.Cu") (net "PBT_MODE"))
 (segment (start 119.69 78.98) (end 113.85 84.82) (width 0.2) (layer "F.Cu") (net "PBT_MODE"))
 (segment (start 134.55 81.86) (end 132.69 80) (width 0.2) (layer "F.Cu") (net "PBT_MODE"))
 (segment (start 126.75 99.5) (end 133.25 99.5) (width 0.2) (layer "F.Cu") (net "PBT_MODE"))
 (segment (start 131.67 78.98) (end 119.69 78.98) (width 0.2) (layer "F.Cu") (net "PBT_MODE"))
 (segment (start 133.25 99.5) (end 134.55 98.2) (width 0.2) (layer "F.Cu") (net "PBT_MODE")))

